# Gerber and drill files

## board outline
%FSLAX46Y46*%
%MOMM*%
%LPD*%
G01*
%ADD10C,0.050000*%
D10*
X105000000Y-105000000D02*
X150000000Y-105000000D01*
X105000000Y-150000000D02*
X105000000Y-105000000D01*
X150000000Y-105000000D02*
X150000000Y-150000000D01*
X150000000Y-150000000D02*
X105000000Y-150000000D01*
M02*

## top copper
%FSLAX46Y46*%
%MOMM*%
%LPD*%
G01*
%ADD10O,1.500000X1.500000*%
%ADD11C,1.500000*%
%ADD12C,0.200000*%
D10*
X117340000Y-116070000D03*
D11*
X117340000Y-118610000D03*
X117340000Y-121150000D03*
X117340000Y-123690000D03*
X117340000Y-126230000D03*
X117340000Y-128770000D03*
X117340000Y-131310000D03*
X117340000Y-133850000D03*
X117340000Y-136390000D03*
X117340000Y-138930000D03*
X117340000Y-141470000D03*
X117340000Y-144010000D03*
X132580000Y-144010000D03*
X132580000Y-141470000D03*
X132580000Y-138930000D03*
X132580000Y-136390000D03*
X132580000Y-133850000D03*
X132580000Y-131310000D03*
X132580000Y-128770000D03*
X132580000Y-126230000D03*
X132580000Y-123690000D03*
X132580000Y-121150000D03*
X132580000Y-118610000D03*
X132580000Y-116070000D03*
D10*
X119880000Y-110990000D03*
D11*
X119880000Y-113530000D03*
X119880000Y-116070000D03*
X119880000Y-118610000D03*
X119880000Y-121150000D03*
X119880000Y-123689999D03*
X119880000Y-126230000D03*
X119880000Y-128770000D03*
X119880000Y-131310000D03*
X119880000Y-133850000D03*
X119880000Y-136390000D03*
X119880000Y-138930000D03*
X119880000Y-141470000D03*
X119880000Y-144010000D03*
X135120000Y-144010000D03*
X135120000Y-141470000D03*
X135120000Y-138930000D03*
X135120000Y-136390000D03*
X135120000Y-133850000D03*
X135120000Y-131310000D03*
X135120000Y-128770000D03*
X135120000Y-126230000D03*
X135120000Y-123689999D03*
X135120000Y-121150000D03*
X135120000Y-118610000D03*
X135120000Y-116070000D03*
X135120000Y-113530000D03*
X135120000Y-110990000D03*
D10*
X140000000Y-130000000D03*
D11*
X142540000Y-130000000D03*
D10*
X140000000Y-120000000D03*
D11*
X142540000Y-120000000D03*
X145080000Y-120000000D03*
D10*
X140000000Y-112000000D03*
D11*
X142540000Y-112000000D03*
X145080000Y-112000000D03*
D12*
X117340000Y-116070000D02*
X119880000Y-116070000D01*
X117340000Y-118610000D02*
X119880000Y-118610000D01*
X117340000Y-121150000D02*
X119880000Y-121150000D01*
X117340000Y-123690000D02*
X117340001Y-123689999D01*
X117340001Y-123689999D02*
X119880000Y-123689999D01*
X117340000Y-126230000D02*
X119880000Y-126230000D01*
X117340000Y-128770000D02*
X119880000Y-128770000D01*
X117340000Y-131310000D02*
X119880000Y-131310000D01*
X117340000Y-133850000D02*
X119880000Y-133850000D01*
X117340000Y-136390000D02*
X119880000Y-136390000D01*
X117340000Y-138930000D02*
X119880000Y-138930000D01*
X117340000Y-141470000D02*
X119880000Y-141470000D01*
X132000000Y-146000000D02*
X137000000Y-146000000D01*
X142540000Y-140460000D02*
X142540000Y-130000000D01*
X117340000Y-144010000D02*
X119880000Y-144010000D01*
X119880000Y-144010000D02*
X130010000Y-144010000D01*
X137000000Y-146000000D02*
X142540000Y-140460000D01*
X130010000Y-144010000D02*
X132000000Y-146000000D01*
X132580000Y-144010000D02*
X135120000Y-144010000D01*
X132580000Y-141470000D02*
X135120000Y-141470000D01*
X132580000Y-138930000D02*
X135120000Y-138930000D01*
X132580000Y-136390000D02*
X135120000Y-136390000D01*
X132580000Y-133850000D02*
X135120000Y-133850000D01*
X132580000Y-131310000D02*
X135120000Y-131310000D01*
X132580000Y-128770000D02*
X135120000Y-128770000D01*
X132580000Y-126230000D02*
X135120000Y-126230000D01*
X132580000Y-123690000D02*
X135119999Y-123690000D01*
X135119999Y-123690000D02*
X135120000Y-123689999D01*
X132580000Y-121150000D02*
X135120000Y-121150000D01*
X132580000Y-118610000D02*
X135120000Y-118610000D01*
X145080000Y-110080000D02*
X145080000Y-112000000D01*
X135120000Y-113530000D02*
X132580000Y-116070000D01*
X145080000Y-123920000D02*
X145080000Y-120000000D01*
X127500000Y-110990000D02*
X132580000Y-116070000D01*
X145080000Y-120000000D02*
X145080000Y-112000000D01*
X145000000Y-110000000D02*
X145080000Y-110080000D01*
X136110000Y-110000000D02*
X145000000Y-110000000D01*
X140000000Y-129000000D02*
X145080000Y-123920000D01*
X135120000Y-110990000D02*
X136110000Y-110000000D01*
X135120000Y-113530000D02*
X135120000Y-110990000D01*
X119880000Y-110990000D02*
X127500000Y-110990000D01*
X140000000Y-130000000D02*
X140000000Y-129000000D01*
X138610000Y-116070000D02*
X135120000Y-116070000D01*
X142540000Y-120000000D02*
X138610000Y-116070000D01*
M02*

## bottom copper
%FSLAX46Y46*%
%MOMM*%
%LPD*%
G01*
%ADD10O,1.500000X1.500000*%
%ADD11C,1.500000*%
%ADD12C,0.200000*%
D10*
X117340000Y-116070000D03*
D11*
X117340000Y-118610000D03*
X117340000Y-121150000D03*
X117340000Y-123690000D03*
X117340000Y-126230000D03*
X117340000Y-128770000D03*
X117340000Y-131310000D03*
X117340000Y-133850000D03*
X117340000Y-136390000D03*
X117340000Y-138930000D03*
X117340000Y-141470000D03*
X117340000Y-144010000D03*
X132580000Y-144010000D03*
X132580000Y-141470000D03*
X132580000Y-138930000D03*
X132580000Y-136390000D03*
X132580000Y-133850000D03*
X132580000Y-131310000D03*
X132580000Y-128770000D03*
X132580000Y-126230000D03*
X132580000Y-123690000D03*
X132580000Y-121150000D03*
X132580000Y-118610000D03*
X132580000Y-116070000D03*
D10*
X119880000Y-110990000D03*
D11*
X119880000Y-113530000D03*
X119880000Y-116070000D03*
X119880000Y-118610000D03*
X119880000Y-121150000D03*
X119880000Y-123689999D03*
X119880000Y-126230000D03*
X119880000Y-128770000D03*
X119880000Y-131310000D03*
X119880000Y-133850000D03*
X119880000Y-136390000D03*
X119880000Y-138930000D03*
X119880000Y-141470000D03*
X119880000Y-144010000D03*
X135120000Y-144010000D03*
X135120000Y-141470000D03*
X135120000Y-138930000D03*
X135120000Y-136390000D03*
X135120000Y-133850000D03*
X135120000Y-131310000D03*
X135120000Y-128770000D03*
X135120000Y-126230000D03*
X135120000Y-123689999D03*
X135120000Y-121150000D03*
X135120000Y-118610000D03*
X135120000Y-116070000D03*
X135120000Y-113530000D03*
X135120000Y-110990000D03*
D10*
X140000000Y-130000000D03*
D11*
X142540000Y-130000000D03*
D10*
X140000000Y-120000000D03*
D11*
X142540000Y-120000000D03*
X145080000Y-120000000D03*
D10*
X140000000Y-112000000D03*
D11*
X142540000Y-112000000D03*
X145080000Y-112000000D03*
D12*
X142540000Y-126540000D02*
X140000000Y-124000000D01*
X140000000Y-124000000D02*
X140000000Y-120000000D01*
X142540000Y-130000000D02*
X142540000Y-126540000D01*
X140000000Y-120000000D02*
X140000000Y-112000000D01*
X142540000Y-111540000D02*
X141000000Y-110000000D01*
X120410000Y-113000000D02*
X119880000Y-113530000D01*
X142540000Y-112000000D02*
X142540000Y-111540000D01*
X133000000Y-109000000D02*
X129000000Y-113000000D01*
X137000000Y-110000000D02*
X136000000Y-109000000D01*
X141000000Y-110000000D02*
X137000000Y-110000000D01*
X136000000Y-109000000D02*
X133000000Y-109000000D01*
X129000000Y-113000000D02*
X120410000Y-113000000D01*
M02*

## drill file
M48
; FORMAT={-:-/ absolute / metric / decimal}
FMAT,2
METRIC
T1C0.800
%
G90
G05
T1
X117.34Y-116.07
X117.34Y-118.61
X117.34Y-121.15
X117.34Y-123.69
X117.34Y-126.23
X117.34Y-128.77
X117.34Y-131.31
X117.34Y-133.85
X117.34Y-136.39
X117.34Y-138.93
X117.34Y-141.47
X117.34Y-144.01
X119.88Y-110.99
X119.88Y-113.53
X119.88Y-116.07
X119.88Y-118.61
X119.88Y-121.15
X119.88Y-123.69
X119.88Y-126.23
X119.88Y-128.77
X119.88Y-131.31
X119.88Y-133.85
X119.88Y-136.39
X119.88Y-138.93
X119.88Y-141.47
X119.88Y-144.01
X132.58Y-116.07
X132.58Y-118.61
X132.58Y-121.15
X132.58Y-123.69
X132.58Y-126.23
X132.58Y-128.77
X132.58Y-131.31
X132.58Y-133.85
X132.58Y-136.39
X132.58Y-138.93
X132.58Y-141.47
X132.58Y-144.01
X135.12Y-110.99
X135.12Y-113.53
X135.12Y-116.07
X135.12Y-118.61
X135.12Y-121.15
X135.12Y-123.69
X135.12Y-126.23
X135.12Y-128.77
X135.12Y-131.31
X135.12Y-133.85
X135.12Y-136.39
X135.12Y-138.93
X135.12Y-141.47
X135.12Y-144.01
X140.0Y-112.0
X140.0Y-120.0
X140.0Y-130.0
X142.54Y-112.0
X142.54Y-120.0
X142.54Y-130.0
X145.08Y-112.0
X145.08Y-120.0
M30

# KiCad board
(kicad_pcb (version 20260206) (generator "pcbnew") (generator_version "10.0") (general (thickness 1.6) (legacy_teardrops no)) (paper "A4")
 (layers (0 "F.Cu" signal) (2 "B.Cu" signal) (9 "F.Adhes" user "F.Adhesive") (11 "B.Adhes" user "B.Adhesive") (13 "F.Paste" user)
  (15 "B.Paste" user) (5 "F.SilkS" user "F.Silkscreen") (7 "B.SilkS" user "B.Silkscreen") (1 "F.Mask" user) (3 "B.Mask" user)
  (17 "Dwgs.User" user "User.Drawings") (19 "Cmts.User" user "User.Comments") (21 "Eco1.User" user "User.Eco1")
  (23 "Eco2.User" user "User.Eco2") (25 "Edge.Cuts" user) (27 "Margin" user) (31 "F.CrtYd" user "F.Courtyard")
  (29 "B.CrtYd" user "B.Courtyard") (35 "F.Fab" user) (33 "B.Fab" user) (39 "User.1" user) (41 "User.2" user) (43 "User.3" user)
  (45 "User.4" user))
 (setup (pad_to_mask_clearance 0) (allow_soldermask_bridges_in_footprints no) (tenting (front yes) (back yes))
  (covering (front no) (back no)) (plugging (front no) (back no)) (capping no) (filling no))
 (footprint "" (layer "F.Cu") (at 100 100)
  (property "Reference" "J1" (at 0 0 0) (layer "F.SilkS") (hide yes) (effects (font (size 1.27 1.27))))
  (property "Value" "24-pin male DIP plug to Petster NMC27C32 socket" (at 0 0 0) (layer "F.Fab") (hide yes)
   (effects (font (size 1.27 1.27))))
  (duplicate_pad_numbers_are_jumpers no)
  (pad "1" thru_hole oval (at 17.34 16.07) (size 1.5 1.5) (drill 0.8) (layers "*.Cu" "*.Mask") (remove_unused_layers no) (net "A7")
   (thermal_bridge_angle 45))
  (pad "2" thru_hole circle (at 17.34 18.61) (size 1.5 1.5) (drill 0.8) (layers "*.Cu" "*.Mask") (remove_unused_layers no) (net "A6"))
  (pad "3" thru_hole circle (at 17.34 21.15) (size 1.5 1.5) (drill 0.8) (layers "*.Cu" "*.Mask") (remove_unused_layers no) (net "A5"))
  (pad "4" thru_hole circle (at 17.34 23.69) (size 1.5 1.5) (drill 0.8) (layers "*.Cu" "*.Mask") (remove_unused_layers no) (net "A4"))
  (pad "5" thru_hole circle (at 17.34 26.23) (size 1.5 1.5) (drill 0.8) (layers "*.Cu" "*.Mask") (remove_unused_layers no) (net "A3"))
  (pad "6" thru_hole circle (at 17.34 28.77) (size 1.5 1.5) (drill 0.8) (layers "*.Cu" "*.Mask") (remove_unused_layers no) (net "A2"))
  (pad "7" thru_hole circle (at 17.34 31.31) (size 1.5 1.5) (drill 0.8) (layers "*.Cu" "*.Mask") (remove_unused_layers no) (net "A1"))
  (pad "8" thru_hole circle (at 17.34 33.85) (size 1.5 1.5) (drill 0.8) (layers "*.Cu" "*.Mask") (remove_unused_layers no) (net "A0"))
  (pad "9" thru_hole circle (at 17.34 36.39) (size 1.5 1.5) (drill 0.8) (layers "*.Cu" "*.Mask") (remove_unused_layers no) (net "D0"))
  (pad "10" thru_hole circle (at 17.34 38.93) (size 1.5 1.5) (drill 0.8) (layers "*.Cu" "*.Mask") (remove_unused_layers no) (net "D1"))
  (pad "11" thru_hole circle (at 17.34 41.47) (size 1.5 1.5) (drill 0.8) (layers "*.Cu" "*.Mask") (remove_unused_layers no) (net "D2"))
  (pad "12" thru_hole circle (at 17.34 44.01) (size 1.5 1.5) (drill 0.8) (layers "*.Cu" "*.Mask") (remove_unused_layers no) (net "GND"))
  (pad "13" thru_hole circle (at 32.58 44.01) (size 1.5 1.5) (drill 0.8) (layers "*.Cu" "*.Mask") (remove_unused_layers no) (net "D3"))
  (pad "14" thru_hole circle (at 32.58 41.47) (size 1.5 1.5) (drill 0.8) (layers "*.Cu" "*.Mask") (remove_unused_layers no) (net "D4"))
  (pad "15" thru_hole circle (at 32.58 38.93) (size 1.5 1.5) (drill 0.8) (layers "*.Cu" "*.Mask") (remove_unused_layers no) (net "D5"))
  (pad "16" thru_hole circle (at 32.58 36.39) (size 1.5 1.5) (drill 0.8) (layers "*.Cu" "*.Mask") (remove_unused_layers no) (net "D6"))
  (pad "17" thru_hole circle (at 32.58 33.85) (size 1.5 1.5) (drill 0.8) (layers "*.Cu" "*.Mask") (remove_unused_layers no) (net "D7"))
  (pad "18" thru_hole circle (at 32.58 31.31) (size 1.5 1.5) (drill 0.8) (layers "*.Cu" "*.Mask") (remove_unused_layers no) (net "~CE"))
  (pad "19" thru_hole circle (at 32.58 28.77) (size 1.5 1.5) (drill 0.8) (layers "*.Cu" "*.Mask") (remove_unused_layers no) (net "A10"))
  (pad "20" thru_hole circle (at 32.58 26.23) (size 1.5 1.5) (drill 0.8) (layers "*.Cu" "*.Mask") (remove_unused_layers no) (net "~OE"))
  (pad "21" thru_hole circle (at 32.58 23.69) (size 1.5 1.5) (drill 0.8) (layers "*.Cu" "*.Mask") (remove_unused_layers no) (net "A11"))
  (pad "22" thru_hole circle (at 32.58 21.15) (size 1.5 1.5) (drill 0.8) (layers "*.Cu" "*.Mask") (remove_unused_layers no) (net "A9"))
  (pad "23" thru_hole circle (at 32.58 18.61) (size 1.5 1.5) (drill 0.8) (layers "*.Cu" "*.Mask") (remove_unused_layers no) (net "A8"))
  (pad "24" thru_hole circle (at 32.58 16.07) (size 1.5 1.5) (drill 0.8) (layers "*.Cu" "*.Mask") (remove_unused_layers no) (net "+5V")))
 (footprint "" (layer "F.Cu") (at 100 100)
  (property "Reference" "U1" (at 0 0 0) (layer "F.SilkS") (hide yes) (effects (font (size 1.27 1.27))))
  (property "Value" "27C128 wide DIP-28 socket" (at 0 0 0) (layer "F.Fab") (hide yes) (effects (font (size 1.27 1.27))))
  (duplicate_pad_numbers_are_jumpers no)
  (pad "1" thru_hole oval (at 19.88 10.99) (size 1.5 1.5) (drill 0.8) (layers "*.Cu" "*.Mask") (remove_unused_layers no) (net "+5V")
   (thermal_bridge_angle 45))
  (pad "2" thru_hole circle (at 19.88 13.53) (size 1.5 1.5) (drill 0.8) (layers "*.Cu" "*.Mask") (remove_unused_layers no) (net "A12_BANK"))
  (pad "3" thru_hole circle (at 19.88 16.07) (size 1.5 1.5) (drill 0.8) (layers "*.Cu" "*.Mask") (remove_unused_layers no) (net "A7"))
  (pad "4" thru_hole circle (at 19.88 18.61) (size 1.5 1.5) (drill 0.8) (layers "*.Cu" "*.Mask") (remove_unused_layers no) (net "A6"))
  (pad "5" thru_hole circle (at 19.88 21.15) (size 1.5 1.5) (drill 0.8) (layers "*.Cu" "*.Mask") (remove_unused_layers no) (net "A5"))
  (pad "6" thru_hole circle (at 19.88 23.689999) (size 1.5 1.5) (drill 0.8) (layers "*.Cu" "*.Mask") (remove_unused_layers no) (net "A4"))
  (pad "7" thru_hole circle (at 19.88 26.23) (size 1.5 1.5) (drill 0.8) (layers "*.Cu" "*.Mask") (remove_unused_layers no) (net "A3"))
  (pad "8" thru_hole circle (at 19.88 28.77) (size 1.5 1.5) (drill 0.8) (layers "*.Cu" "*.Mask") (remove_unused_layers no) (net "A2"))
  (pad "9" thru_hole circle (at 19.88 31.31) (size 1.5 1.5) (drill 0.8) (layers "*.Cu" "*.Mask") (remove_unused_layers no) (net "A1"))
  (pad "10" thru_hole circle (at 19.88 33.85) (size 1.5 1.5) (drill 0.8) (layers "*.Cu" "*.Mask") (remove_unused_layers no) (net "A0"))
  (pad "11" thru_hole circle (at 19.88 36.39) (size 1.5 1.5) (drill 0.8) (layers "*.Cu" "*.Mask") (remove_unused_layers no) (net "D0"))
  (pad "12" thru_hole circle (at 19.88 38.93) (size 1.5 1.5) (drill 0.8) (layers "*.Cu" "*.Mask") (remove_unused_layers no) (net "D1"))
  (pad "13" thru_hole circle (at 19.88 41.47) (size 1.5 1.5) (drill 0.8) (layers "*.Cu" "*.Mask") (remove_unused_layers no) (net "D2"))
  (pad "14" thru_hole circle (at 19.88 44.01) (size 1.5 1.5) (drill 0.8) (layers "*.Cu" "*.Mask") (remove_unused_layers no) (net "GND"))
  (pad "15" thru_hole circle (at 35.12 44.01) (size 1.5 1.5) (drill 0.8) (layers "*.Cu" "*.Mask") (remove_unused_layers no) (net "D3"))
  (pad "16" thru_hole circle (at 35.12 41.47) (size 1.5 1.5) (drill 0.8) (layers "*.Cu" "*.Mask") (remove_unused_layers no) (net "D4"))
  (pad "17" thru_hole circle (at 35.12 38.93) (size 1.5 1.5) (drill 0.8) (layers "*.Cu" "*.Mask") (remove_unused_layers no) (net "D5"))
  (pad "18" thru_hole circle (at 35.12 36.39) (size 1.5 1.5) (drill 0.8) (layers "*.Cu" "*.Mask") (remove_unused_layers no) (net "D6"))
  (pad "19" thru_hole circle (at 35.12 33.85) (size 1.5 1.5) (drill 0.8) (layers "*.Cu" "*.Mask") (remove_unused_layers no) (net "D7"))
  (pad "20" thru_hole circle (at 35.12 31.31) (size 1.5 1.5) (drill 0.8) (layers "*.Cu" "*.Mask") (remove_unused_layers no) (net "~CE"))
  (pad "21" thru_hole circle (at 35.12 28.77) (size 1.5 1.5) (drill 0.8) (layers "*.Cu" "*.Mask") (remove_unused_layers no) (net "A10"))
  (pad "22" thru_hole circle (at 35.12 26.23) (size 1.5 1.5) (drill 0.8) (layers "*.Cu" "*.Mask") (remove_unused_layers no) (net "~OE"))
  (pad "23" thru_hole circle (at 35.12 23.689999) (size 1.5 1.5) (drill 0.8) (layers "*.Cu" "*.Mask") (remove_unused_layers no) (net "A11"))
  (pad "24" thru_hole circle (at 35.12 21.15) (size 1.5 1.5) (drill 0.8) (layers "*.Cu" "*.Mask") (remove_unused_layers no) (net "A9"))
  (pad "25" thru_hole circle (at 35.12 18.61) (size 1.5 1.5) (drill 0.8) (layers "*.Cu" "*.Mask") (remove_unused_layers no) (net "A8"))
  (pad "26" thru_hole circle (at 35.12 16.07) (size 1.5 1.5) (drill 0.8) (layers "*.Cu" "*.Mask") (remove_unused_layers no) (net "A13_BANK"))
  (pad "27" thru_hole circle (at 35.12 13.53) (size 1.5 1.5) (drill 0.8) (layers "*.Cu" "*.Mask") (remove_unused_layers no) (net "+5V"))
  (pad "28" thru_hole circle (at 35.12 10.99) (size 1.5 1.5) (drill 0.8) (layers "*.Cu" "*.Mask") (remove_unused_layers no) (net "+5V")))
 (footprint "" (layer "F.Cu") (at 100 100)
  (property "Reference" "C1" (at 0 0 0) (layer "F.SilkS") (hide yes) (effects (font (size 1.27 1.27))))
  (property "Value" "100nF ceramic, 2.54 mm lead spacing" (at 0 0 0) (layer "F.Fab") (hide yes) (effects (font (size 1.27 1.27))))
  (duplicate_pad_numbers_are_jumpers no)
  (pad "1" thru_hole oval (at 40 30) (size 1.5 1.5) (drill 0.8) (layers "*.Cu" "*.Mask") (remove_unused_layers no) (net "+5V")
   (thermal_bridge_angle 45))
  (pad "2" thru_hole circle (at 42.54 30) (size 1.5 1.5) (drill 0.8) (layers "*.Cu" "*.Mask") (remove_unused_layers no) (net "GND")))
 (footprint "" (layer "F.Cu") (at 100 100)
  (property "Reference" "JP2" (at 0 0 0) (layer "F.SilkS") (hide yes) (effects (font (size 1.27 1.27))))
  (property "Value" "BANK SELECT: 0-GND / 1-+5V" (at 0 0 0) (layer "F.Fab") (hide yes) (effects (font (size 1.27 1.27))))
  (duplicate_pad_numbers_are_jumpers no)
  (pad "1" thru_hole oval (at 40 20) (size 1.5 1.5) (drill 0.8) (layers "*.Cu" "*.Mask") (remove_unused_layers no) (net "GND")
   (thermal_bridge_angle 45))
  (pad "2" thru_hole circle (at 42.54 20) (size 1.5 1.5) (drill 0.8) (layers "*.Cu" "*.Mask") (remove_unused_layers no) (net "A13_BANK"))
  (pad "3" thru_hole circle (at 45.08 20) (size 1.5 1.5) (drill 0.8) (layers "*.Cu" "*.Mask") (remove_unused_layers no) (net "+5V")))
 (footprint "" (layer "F.Cu") (at 100 100)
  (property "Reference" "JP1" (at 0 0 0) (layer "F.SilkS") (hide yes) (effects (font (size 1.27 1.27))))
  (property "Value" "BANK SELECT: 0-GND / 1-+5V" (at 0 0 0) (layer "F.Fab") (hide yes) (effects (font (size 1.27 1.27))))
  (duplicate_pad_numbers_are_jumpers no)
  (pad "1" thru_hole oval (at 40 12) (size 1.5 1.5) (drill 0.8) (layers "*.Cu" "*.Mask") (remove_unused_layers no) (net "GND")
   (thermal_bridge_angle 45))
  (pad "2" thru_hole circle (at 42.54 12) (size 1.5 1.5) (drill 0.8) (layers "*.Cu" "*.Mask") (remove_unused_layers no) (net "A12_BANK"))
  (pad "3" thru_hole circle (at 45.08 12) (size 1.5 1.5) (drill 0.8) (layers "*.Cu" "*.Mask") (remove_unused_layers no) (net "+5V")))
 (gr_line (start 105 105) (end 150 105) (stroke (width 0.05) (type default)) (layer "Edge.Cuts"))
 (gr_line (start 105 150) (end 105 105) (stroke (width 0.05) (type default)) (layer "Edge.Cuts"))
 (gr_line (start 150 105) (end 150 150) (stroke (width 0.05) (type default)) (layer "Edge.Cuts"))
 (gr_line (start 150 150) (end 105 150) (stroke (width 0.05) (type default)) (layer "Edge.Cuts"))
 (segment (start 117.34 116.07) (end 119.88 116.07) (width 0.2) (layer "F.Cu") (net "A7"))
 (segment (start 117.34 118.61) (end 119.88 118.61) (width 0.2) (layer "F.Cu") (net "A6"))
 (segment (start 117.34 121.15) (end 119.88 121.15) (width 0.2) (layer "F.Cu") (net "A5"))
 (segment (start 117.34 123.69) (end 117.340001 123.689999) (width 0.2) (layer "F.Cu") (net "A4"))
 (segment (start 117.340001 123.689999) (end 119.88 123.689999) (width 0.2) (layer "F.Cu") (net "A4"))
 (segment (start 117.34 126.23) (end 119.88 126.23) (width 0.2) (layer "F.Cu") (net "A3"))
 (segment (start 117.34 128.77) (end 119.88 128.77) (width 0.2) (layer "F.Cu") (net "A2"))
 (segment (start 117.34 131.31) (end 119.88 131.31) (width 0.2) (layer "F.Cu") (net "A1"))
 (segment (start 117.34 133.85) (end 119.88 133.85) (width 0.2) (layer "F.Cu") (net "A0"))
 (segment (start 117.34 136.39) (end 119.88 136.39) (width 0.2) (layer "F.Cu") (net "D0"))
 (segment (start 117.34 138.93) (end 119.88 138.93) (width 0.2) (layer "F.Cu") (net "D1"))
 (segment (start 117.34 141.47) (end 119.88 141.47) (width 0.2) (layer "F.Cu") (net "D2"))
 (segment (start 132 146) (end 137 146) (width 0.2) (layer "F.Cu") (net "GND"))
 (segment (start 142.54 140.46) (end 142.54 130) (width 0.2) (layer "F.Cu") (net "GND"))
 (segment (start 117.34 144.01) (end 119.88 144.01) (width 0.2) (layer "F.Cu") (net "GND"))
 (segment (start 119.88 144.01) (end 130.01 144.01) (width 0.2) (layer "F.Cu") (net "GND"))
 (segment (start 137 146) (end 142.54 140.46) (width 0.2) (layer "F.Cu") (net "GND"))
 (segment (start 130.01 144.01) (end 132 146) (width 0.2) (layer "F.Cu") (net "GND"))
 (segment (start 142.54 126.54) (end 140 124) (width 0.2) (layer "B.Cu") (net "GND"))
 (segment (start 140 124) (end 140 120) (width 0.2) (layer "B.Cu") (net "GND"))
 (segment (start 142.54 130) (end 142.54 126.54) (width 0.2) (layer "B.Cu") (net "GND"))
 (segment (start 140 120) (end 140 112) (width 0.2) (layer "B.Cu") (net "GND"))
 (segment (start 132.58 144.01) (end 135.12 144.01) (width 0.2) (layer "F.Cu") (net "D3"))
 (segment (start 132.58 141.47) (end 135.12 141.47) (width 0.2) (layer "F.Cu") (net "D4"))
 (segment (start 132.58 138.93) (end 135.12 138.93) (width 0.2) (layer "F.Cu") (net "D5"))
 (segment (start 132.58 136.39) (end 135.12 136.39) (width 0.2) (layer "F.Cu") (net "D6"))
 (segment (start 132.58 133.85) (end 135.12 133.85) (width 0.2) (layer "F.Cu") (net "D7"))
 (segment (start 132.58 131.31) (end 135.12 131.31) (width 0.2) (layer "F.Cu") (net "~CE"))
 (segment (start 132.58 128.77) (end 135.12 128.77) (width 0.2) (layer "F.Cu") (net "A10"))
 (segment (start 132.58 126.23) (end 135.12 126.23) (width 0.2) (layer "F.Cu") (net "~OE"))
 (segment (start 132.58 123.69) (end 135.119999 123.69) (width 0.2) (layer "F.Cu") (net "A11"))
 (segment (start 135.119999 123.69) (end 135.12 123.689999) (width 0.2) (layer "F.Cu") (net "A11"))
 (segment (start 132.58 121.15) (end 135.12 121.15) (width 0.2) (layer "F.Cu") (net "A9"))
 (segment (start 132.58 118.61) (end 135.12 118.61) (width 0.2) (layer "F.Cu") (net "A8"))
 (segment (start 145.08 110.08) (end 145.08 112) (width 0.2) (layer "F.Cu") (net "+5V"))
 (segment (start 135.12 113.53) (end 132.58 116.07) (width 0.2) (layer "F.Cu") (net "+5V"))
 (segment (start 145.08 123.92) (end 145.08 120) (width 0.2) (layer "F.Cu") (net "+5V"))
 (segment (start 127.5 110.99) (end 132.58 116.07) (width 0.2) (layer "F.Cu") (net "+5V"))
 (segment (start 145.08 120) (end 145.08 112) (width 0.2) (layer "F.Cu") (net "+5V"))
 (segment (start 145 110) (end 145.08 110.08) (width 0.2) (layer "F.Cu") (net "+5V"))
 (segment (start 136.11 110) (end 145 110) (width 0.2) (layer "F.Cu") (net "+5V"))
 (segment (start 140 129) (end 145.08 123.92) (width 0.2) (layer "F.Cu") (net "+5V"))
 (segment (start 135.12 110.99) (end 136.11 110) (width 0.2) (layer "F.Cu") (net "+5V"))
 (segment (start 135.12 113.53) (end 135.12 110.99) (width 0.2) (layer "F.Cu") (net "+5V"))
 (segment (start 119.88 110.99) (end 127.5 110.99) (width 0.2) (layer "F.Cu") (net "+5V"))
 (segment (start 140 130) (end 140 129) (width 0.2) (layer "F.Cu") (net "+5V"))
 (segment (start 142.54 111.54) (end 141 110) (width 0.2) (layer "B.Cu") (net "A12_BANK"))
 (segment (start 120.41 113) (end 119.88 113.53) (width 0.2) (layer "B.Cu") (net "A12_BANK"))
 (segment (start 142.54 112) (end 142.54 111.54) (width 0.2) (layer "B.Cu") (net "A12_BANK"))
 (segment (start 133 109) (end 129 113) (width 0.2) (layer "B.Cu") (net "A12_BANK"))
 (segment (start 137 110) (end 136 109) (width 0.2) (layer "B.Cu") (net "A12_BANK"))
 (segment (start 141 110) (end 137 110) (width 0.2) (layer "B.Cu") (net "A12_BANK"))
 (segment (start 136 109) (end 133 109) (width 0.2) (layer "B.Cu") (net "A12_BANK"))
 (segment (start 129 113) (end 120.41 113) (width 0.2) (layer "B.Cu") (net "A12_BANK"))
 (segment (start 138.61 116.07) (end 135.12 116.07) (width 0.2) (layer "F.Cu") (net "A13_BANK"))
 (segment (start 142.54 120) (end 138.61 116.07) (width 0.2) (layer "F.Cu") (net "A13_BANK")))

